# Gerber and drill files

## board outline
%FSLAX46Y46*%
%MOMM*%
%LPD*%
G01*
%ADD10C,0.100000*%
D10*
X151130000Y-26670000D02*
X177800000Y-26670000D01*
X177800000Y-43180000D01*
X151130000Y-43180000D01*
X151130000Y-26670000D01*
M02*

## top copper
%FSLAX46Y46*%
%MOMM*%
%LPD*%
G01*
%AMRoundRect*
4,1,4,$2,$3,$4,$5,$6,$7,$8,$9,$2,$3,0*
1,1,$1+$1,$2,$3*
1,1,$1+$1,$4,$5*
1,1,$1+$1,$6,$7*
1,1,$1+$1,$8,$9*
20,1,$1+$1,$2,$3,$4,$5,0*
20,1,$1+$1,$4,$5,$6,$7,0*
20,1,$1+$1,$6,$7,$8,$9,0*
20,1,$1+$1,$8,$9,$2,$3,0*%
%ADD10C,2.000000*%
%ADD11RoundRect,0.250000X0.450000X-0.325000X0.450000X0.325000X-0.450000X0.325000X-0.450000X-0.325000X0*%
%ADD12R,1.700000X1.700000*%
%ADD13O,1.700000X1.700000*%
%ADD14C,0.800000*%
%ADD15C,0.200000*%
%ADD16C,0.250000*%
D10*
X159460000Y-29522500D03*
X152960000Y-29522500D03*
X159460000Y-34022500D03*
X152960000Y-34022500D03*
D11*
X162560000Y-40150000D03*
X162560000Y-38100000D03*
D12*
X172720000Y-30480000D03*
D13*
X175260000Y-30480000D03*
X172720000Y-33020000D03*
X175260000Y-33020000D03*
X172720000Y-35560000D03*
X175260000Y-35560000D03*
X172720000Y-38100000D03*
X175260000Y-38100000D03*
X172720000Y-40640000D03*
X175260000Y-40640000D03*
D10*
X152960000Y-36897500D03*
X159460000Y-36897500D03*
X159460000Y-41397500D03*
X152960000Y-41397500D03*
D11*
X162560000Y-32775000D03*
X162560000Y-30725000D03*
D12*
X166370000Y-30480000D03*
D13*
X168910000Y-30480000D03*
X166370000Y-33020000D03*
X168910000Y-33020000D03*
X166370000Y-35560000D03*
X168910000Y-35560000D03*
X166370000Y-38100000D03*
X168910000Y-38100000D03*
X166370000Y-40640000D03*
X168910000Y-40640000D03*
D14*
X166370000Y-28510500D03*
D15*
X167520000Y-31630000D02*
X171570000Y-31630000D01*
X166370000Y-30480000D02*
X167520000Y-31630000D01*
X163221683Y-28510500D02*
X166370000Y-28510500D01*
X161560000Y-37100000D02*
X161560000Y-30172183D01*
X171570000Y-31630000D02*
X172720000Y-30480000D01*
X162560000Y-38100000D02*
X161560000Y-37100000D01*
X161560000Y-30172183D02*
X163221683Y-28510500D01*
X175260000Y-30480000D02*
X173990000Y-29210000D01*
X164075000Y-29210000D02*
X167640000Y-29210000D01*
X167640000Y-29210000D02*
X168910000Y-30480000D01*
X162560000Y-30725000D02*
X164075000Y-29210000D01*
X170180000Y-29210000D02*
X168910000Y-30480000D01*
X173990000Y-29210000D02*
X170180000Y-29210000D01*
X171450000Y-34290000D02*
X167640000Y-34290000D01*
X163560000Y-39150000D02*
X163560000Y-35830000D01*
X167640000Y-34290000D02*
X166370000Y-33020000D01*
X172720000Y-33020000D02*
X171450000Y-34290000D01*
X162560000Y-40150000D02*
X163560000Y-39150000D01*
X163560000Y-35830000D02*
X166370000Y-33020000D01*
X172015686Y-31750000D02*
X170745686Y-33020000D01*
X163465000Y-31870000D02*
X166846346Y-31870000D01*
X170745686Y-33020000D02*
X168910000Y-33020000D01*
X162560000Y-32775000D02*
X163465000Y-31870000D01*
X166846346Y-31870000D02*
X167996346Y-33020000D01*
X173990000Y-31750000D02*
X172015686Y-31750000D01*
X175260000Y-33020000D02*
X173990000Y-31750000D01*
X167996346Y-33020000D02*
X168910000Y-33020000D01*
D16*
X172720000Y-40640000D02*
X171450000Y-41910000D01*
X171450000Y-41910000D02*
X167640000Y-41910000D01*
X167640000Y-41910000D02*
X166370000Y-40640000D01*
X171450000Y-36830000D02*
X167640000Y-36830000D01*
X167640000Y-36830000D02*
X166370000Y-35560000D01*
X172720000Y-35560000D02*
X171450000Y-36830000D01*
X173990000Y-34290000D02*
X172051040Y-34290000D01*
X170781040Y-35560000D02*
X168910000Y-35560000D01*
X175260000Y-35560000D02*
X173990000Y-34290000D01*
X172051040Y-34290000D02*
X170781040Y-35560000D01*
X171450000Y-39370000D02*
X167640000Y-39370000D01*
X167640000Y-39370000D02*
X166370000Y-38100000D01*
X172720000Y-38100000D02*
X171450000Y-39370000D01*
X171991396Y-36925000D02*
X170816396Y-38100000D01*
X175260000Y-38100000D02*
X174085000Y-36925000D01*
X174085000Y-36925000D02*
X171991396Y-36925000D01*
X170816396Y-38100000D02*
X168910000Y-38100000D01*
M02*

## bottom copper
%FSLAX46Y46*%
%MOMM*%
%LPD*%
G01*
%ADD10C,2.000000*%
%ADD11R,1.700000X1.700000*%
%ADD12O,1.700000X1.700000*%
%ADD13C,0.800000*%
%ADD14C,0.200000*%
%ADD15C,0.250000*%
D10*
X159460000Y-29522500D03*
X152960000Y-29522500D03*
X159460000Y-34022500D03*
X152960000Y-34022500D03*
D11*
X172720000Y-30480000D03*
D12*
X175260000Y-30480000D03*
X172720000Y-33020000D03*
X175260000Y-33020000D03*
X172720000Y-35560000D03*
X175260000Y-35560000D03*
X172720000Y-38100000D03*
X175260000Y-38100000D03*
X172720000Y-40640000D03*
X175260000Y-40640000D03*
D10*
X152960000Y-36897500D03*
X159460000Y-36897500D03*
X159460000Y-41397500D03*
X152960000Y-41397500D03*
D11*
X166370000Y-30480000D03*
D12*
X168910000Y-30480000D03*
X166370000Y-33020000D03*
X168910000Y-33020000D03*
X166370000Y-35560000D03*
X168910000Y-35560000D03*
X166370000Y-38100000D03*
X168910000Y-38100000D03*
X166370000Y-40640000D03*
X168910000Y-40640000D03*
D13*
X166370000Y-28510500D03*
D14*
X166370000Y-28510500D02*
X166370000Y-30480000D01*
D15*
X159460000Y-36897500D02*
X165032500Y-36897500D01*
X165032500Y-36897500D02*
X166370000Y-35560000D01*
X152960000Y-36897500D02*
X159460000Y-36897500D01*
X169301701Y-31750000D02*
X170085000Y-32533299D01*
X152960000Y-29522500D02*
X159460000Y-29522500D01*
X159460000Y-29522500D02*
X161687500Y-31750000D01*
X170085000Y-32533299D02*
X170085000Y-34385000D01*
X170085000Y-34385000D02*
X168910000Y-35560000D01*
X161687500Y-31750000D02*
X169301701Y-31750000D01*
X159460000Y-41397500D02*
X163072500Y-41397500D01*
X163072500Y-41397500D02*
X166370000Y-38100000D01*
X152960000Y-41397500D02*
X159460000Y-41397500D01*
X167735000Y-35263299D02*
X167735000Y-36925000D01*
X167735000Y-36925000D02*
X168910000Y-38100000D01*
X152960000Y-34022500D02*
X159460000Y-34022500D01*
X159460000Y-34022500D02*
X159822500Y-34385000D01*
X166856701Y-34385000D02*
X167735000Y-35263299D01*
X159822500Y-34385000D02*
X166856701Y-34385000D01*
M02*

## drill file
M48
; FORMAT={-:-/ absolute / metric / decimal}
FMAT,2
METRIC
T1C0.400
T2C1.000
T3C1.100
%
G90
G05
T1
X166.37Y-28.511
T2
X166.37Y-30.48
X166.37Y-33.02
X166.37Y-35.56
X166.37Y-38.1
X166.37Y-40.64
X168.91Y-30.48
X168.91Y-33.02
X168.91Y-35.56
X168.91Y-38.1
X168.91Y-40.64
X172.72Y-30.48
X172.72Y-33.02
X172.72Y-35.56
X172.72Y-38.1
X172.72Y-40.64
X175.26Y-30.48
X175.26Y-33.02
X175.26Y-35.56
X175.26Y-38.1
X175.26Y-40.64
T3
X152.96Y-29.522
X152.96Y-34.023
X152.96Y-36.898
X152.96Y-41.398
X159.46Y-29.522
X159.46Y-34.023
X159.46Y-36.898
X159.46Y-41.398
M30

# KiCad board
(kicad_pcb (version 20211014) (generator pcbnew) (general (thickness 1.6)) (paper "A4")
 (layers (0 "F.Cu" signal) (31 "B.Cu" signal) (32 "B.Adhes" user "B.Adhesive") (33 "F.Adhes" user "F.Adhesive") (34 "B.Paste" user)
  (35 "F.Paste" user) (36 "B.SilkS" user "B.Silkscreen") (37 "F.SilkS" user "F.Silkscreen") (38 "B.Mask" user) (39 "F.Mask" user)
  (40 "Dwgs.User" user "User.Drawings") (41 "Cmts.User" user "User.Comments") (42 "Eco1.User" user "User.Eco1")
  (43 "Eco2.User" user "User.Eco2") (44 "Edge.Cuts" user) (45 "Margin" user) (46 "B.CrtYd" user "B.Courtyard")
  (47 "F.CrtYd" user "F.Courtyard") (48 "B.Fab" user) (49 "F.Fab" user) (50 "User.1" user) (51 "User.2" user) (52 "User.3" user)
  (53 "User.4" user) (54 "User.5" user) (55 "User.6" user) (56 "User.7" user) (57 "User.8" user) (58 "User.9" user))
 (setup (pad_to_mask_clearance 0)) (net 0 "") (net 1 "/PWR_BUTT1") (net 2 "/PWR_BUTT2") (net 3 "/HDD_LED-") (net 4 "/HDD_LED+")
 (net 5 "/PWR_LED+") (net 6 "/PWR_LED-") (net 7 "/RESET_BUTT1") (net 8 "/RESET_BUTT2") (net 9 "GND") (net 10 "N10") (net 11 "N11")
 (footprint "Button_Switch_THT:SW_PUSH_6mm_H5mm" (layer "F.Cu") (at 152.96 29.5225)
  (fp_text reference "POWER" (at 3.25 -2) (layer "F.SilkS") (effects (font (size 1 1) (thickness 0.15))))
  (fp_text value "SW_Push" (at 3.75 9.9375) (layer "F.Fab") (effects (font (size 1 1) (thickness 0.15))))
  (pad "1" thru_hole circle (at 6.5 0 90) (size 2 2) (drill 1.1) (layers *.Cu *.Mask) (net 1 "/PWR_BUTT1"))
  (pad "1" thru_hole circle (at 0 0 90) (size 2 2) (drill 1.1) (layers *.Cu *.Mask) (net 1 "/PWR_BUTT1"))
  (pad "2" thru_hole circle (at 6.5 4.5 90) (size 2 2) (drill 1.1) (layers *.Cu *.Mask) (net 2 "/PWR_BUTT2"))
  (pad "2" thru_hole circle (at 0 4.5 90) (size 2 2) (drill 1.1) (layers *.Cu *.Mask) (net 2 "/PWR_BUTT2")))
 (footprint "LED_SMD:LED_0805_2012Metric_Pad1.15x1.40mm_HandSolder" (layer "F.Cu") (at 162.56 39.125 90)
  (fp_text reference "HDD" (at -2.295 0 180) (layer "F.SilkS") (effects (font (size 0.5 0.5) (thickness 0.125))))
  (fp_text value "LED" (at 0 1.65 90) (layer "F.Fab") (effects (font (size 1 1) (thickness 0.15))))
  (pad "1" smd roundrect (at -1.025 0 90) (size 1.15 1.4) (layers "F.Cu" "F.Paste" "F.Mask") (roundrect_rratio 0.217391) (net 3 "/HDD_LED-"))
  (pad "2" smd roundrect (at 1.025 0 90) (size 1.15 1.4) (layers "F.Cu" "F.Paste" "F.Mask") (roundrect_rratio 0.217391) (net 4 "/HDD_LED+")))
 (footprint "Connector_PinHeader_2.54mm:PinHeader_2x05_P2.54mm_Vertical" (layer "F.Cu") (at 172.72 30.48)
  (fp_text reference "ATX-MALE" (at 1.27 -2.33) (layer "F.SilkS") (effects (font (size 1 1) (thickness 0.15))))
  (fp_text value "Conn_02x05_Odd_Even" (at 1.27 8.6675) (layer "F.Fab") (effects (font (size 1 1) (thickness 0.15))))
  (pad "1" thru_hole rect (at 0 0) (size 1.7 1.7) (drill 1) (layers *.Cu *.Mask) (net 4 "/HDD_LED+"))
  (pad "2" thru_hole oval (at 2.54 0) (size 1.7 1.7) (drill 1) (layers *.Cu *.Mask) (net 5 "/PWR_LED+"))
  (pad "3" thru_hole oval (at 0 2.54) (size 1.7 1.7) (drill 1) (layers *.Cu *.Mask) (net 3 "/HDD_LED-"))
  (pad "4" thru_hole oval (at 2.54 2.54) (size 1.7 1.7) (drill 1) (layers *.Cu *.Mask) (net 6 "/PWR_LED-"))
  (pad "5" thru_hole oval (at 0 5.08) (size 1.7 1.7) (drill 1) (layers *.Cu *.Mask) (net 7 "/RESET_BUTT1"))
  (pad "6" thru_hole oval (at 2.54 5.08) (size 1.7 1.7) (drill 1) (layers *.Cu *.Mask) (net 1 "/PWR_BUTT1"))
  (pad "7" thru_hole oval (at 0 7.62) (size 1.7 1.7) (drill 1) (layers *.Cu *.Mask) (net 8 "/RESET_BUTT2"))
  (pad "8" thru_hole oval (at 2.54 7.62) (size 1.7 1.7) (drill 1) (layers *.Cu *.Mask) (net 2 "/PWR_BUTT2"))
  (pad "9" thru_hole oval (at 0 10.16) (size 1.7 1.7) (drill 1) (layers *.Cu *.Mask) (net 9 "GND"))
  (pad "10" thru_hole oval (at 2.54 10.16) (size 1.7 1.7) (drill 1) (layers *.Cu *.Mask) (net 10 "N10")))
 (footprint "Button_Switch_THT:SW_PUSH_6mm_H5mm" (layer "F.Cu") (at 152.96 36.8975)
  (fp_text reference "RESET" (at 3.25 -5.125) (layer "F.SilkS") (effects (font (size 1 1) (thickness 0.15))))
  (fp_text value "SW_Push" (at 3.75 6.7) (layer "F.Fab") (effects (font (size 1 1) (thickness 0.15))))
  (pad "1" thru_hole circle (at 0 0 90) (size 2 2) (drill 1.1) (layers *.Cu *.Mask) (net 7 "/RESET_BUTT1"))
  (pad "1" thru_hole circle (at 6.5 0 90) (size 2 2) (drill 1.1) (layers *.Cu *.Mask) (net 7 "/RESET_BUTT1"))
  (pad "2" thru_hole circle (at 6.5 4.5 90) (size 2 2) (drill 1.1) (layers *.Cu *.Mask) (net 8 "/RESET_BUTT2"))
  (pad "2" thru_hole circle (at 0 4.5 90) (size 2 2) (drill 1.1) (layers *.Cu *.Mask) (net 8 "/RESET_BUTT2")))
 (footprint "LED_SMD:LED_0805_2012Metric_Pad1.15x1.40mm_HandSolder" (layer "F.Cu") (at 162.56 31.75 90)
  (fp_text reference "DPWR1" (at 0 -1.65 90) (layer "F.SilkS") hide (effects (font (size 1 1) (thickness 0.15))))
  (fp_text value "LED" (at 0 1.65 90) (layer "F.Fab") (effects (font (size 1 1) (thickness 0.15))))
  (pad "1" smd roundrect (at -1.025 0 90) (size 1.15 1.4) (layers "F.Cu" "F.Paste" "F.Mask") (roundrect_rratio 0.217391) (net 6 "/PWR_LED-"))
  (pad "2" smd roundrect (at 1.025 0 90) (size 1.15 1.4) (layers "F.Cu" "F.Paste" "F.Mask") (roundrect_rratio 0.217391) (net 5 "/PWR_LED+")))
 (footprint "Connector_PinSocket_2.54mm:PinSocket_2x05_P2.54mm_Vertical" (layer "B.Cu") (at 166.37 30.48 180)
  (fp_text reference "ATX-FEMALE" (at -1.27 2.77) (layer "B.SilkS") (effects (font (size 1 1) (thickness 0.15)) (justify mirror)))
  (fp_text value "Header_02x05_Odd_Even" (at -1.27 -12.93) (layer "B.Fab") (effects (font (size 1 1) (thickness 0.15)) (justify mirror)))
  (pad "1" thru_hole rect (at 0 0 180) (size 1.7 1.7) (drill 1) (layers *.Cu *.Mask) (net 4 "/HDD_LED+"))
  (pad "2" thru_hole oval (at -2.54 0 180) (size 1.7 1.7) (drill 1) (layers *.Cu *.Mask) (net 5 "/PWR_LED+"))
  (pad "3" thru_hole oval (at 0 -2.54 180) (size 1.7 1.7) (drill 1) (layers *.Cu *.Mask) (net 3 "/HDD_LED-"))
  (pad "4" thru_hole oval (at -2.54 -2.54 180) (size 1.7 1.7) (drill 1) (layers *.Cu *.Mask) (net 6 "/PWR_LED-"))
  (pad "5" thru_hole oval (at 0 -5.08 180) (size 1.7 1.7) (drill 1) (layers *.Cu *.Mask) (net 7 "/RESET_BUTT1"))
  (pad "6" thru_hole oval (at -2.54 -5.08 180) (size 1.7 1.7) (drill 1) (layers *.Cu *.Mask) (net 1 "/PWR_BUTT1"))
  (pad "7" thru_hole oval (at 0 -7.62 180) (size 1.7 1.7) (drill 1) (layers *.Cu *.Mask) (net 8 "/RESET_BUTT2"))
  (pad "8" thru_hole oval (at -2.54 -7.62 180) (size 1.7 1.7) (drill 1) (layers *.Cu *.Mask) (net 2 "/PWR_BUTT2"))
  (pad "9" thru_hole oval (at 0 -10.16 180) (size 1.7 1.7) (drill 1) (layers *.Cu *.Mask) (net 9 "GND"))
  (pad "10" thru_hole oval (at -2.54 -10.16 180) (size 1.7 1.7) (drill 1) (layers *.Cu *.Mask) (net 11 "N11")))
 (gr_rect (start 177.8 26.67) (end 151.13 43.18) (layer "Edge.Cuts") (width 0.1) (fill none))
 (segment (start 167.52 31.63) (end 171.57 31.63) (width 0.2) (layer "F.Cu") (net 4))
 (segment (start 166.37 30.48) (end 167.52 31.63) (width 0.2) (layer "F.Cu") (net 4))
 (segment (start 163.221683 28.5105) (end 166.37 28.5105) (width 0.2) (layer "F.Cu") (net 4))
 (segment (start 161.56 37.1) (end 161.56 30.172183) (width 0.2) (layer "F.Cu") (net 4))
 (segment (start 171.57 31.63) (end 172.72 30.48) (width 0.2) (layer "F.Cu") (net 4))
 (segment (start 162.56 38.1) (end 161.56 37.1) (width 0.2) (layer "F.Cu") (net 4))
 (segment (start 161.56 30.172183) (end 163.221683 28.5105) (width 0.2) (layer "F.Cu") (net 4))
 (via (at 166.37 28.5105) (size 0.8) (drill 0.4) (layers "F.Cu" "B.Cu") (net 4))
 (segment (start 166.37 28.5105) (end 166.37 30.48) (width 0.2) (layer "B.Cu") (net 4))
 (segment (start 175.26 30.48) (end 173.99 29.21) (width 0.2) (layer "F.Cu") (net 5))
 (segment (start 164.075 29.21) (end 167.64 29.21) (width 0.2) (layer "F.Cu") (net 5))
 (segment (start 167.64 29.21) (end 168.91 30.48) (width 0.2) (layer "F.Cu") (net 5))
 (segment (start 162.56 30.725) (end 164.075 29.21) (width 0.2) (layer "F.Cu") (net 5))
 (segment (start 170.18 29.21) (end 168.91 30.48) (width 0.2) (layer "F.Cu") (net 5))
 (segment (start 173.99 29.21) (end 170.18 29.21) (width 0.2) (layer "F.Cu") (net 5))
 (segment (start 171.45 34.29) (end 167.64 34.29) (width 0.2) (layer "F.Cu") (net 3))
 (segment (start 163.56 39.15) (end 163.56 35.83) (width 0.2) (layer "F.Cu") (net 3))
 (segment (start 167.64 34.29) (end 166.37 33.02) (width 0.2) (layer "F.Cu") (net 3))
 (segment (start 172.72 33.02) (end 171.45 34.29) (width 0.2) (layer "F.Cu") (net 3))
 (segment (start 162.56 40.15) (end 163.56 39.15) (width 0.2) (layer "F.Cu") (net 3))
 (segment (start 163.56 35.83) (end 166.37 33.02) (width 0.2) (layer "F.Cu") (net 3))
 (segment (start 172.015686 31.75) (end 170.745686 33.02) (width 0.2) (layer "F.Cu") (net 6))
 (segment (start 163.465 31.87) (end 166.846346 31.87) (width 0.2) (layer "F.Cu") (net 6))
 (segment (start 170.745686 33.02) (end 168.91 33.02) (width 0.2) (layer "F.Cu") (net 6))
 (segment (start 162.56 32.775) (end 163.465 31.87) (width 0.2) (layer "F.Cu") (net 6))
 (segment (start 166.846346 31.87) (end 167.996346 33.02) (width 0.2) (layer "F.Cu") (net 6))
 (segment (start 173.99 31.75) (end 172.015686 31.75) (width 0.2) (layer "F.Cu") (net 6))
 (segment (start 175.26 33.02) (end 173.99 31.75) (width 0.2) (layer "F.Cu") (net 6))
 (segment (start 167.996346 33.02) (end 168.91 33.02) (width 0.2) (layer "F.Cu") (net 6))
 (segment (start 172.72 40.64) (end 171.45 41.91) (width 0.25) (layer "F.Cu") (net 9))
 (segment (start 171.45 41.91) (end 167.64 41.91) (width 0.25) (layer "F.Cu") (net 9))
 (segment (start 167.64 41.91) (end 166.37 40.64) (width 0.25) (layer "F.Cu") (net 9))
 (segment (start 171.45 36.83) (end 167.64 36.83) (width 0.25) (layer "F.Cu") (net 7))
 (segment (start 167.64 36.83) (end 166.37 35.56) (width 0.25) (layer "F.Cu") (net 7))
 (segment (start 172.72 35.56) (end 171.45 36.83) (width 0.25) (layer "F.Cu") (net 7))
 (segment (start 159.46 36.8975) (end 165.0325 36.8975) (width 0.25) (layer "B.Cu") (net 7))
 (segment (start 165.0325 36.8975) (end 166.37 35.56) (width 0.25) (layer "B.Cu") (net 7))
 (segment (start 152.96 36.8975) (end 159.46 36.8975) (width 0.25) (layer "B.Cu") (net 7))
 (segment (start 173.99 34.29) (end 172.05104 34.29) (width 0.25) (layer "F.Cu") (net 1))
 (segment (start 170.78104 35.56) (end 168.91 35.56) (width 0.25) (layer "F.Cu") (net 1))
 (segment (start 175.26 35.56) (end 173.99 34.29) (width 0.25) (layer "F.Cu") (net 1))
 (segment (start 172.05104 34.29) (end 170.78104 35.56) (width 0.25) (layer "F.Cu") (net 1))
 (segment (start 169.301701 31.75) (end 170.085 32.533299) (width 0.25) (layer "B.Cu") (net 1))
 (segment (start 152.96 29.5225) (end 159.46 29.5225) (width 0.25) (layer "B.Cu") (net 1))
 (segment (start 159.46 29.5225) (end 161.6875 31.75) (width 0.25) (layer "B.Cu") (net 1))
 (segment (start 170.085 32.533299) (end 170.085 34.385) (width 0.25) (layer "B.Cu") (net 1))
 (segment (start 170.085 34.385) (end 168.91 35.56) (width 0.25) (layer "B.Cu") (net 1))
 (segment (start 161.6875 31.75) (end 169.301701 31.75) (width 0.25) (layer "B.Cu") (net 1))
 (segment (start 171.45 39.37) (end 167.64 39.37) (width 0.25) (layer "F.Cu") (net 8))
 (segment (start 167.64 39.37) (end 166.37 38.1) (width 0.25) (layer "F.Cu") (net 8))
 (segment (start 172.72 38.1) (end 171.45 39.37) (width 0.25) (layer "F.Cu") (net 8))
 (segment (start 159.46 41.3975) (end 163.0725 41.3975) (width 0.25) (layer "B.Cu") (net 8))
 (segment (start 163.0725 41.3975) (end 166.37 38.1) (width 0.25) (layer "B.Cu") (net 8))
 (segment (start 152.96 41.3975) (end 159.46 41.3975) (width 0.25) (layer "B.Cu") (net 8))
 (segment (start 171.991396 36.925) (end 170.816396 38.1) (width 0.25) (layer "F.Cu") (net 2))
 (segment (start 175.26 38.1) (end 174.085 36.925) (width 0.25) (layer "F.Cu") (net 2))
 (segment (start 174.085 36.925) (end 171.991396 36.925) (width 0.25) (layer "F.Cu") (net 2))
 (segment (start 170.816396 38.1) (end 168.91 38.1) (width 0.25) (layer "F.Cu") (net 2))
 (segment (start 167.735 35.263299) (end 167.735 36.925) (width 0.25) (layer "B.Cu") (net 2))
 (segment (start 167.735 36.925) (end 168.91 38.1) (width 0.25) (layer "B.Cu") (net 2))
 (segment (start 152.96 34.0225) (end 159.46 34.0225) (width 0.25) (layer "B.Cu") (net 2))
 (segment (start 159.46 34.0225) (end 159.8225 34.385) (width 0.25) (layer "B.Cu") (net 2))
 (segment (start 166.856701 34.385) (end 167.735 35.263299) (width 0.25) (layer "B.Cu") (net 2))
 (segment (start 159.8225 34.385) (end 166.856701 34.385) (width 0.25) (layer "B.Cu") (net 2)))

